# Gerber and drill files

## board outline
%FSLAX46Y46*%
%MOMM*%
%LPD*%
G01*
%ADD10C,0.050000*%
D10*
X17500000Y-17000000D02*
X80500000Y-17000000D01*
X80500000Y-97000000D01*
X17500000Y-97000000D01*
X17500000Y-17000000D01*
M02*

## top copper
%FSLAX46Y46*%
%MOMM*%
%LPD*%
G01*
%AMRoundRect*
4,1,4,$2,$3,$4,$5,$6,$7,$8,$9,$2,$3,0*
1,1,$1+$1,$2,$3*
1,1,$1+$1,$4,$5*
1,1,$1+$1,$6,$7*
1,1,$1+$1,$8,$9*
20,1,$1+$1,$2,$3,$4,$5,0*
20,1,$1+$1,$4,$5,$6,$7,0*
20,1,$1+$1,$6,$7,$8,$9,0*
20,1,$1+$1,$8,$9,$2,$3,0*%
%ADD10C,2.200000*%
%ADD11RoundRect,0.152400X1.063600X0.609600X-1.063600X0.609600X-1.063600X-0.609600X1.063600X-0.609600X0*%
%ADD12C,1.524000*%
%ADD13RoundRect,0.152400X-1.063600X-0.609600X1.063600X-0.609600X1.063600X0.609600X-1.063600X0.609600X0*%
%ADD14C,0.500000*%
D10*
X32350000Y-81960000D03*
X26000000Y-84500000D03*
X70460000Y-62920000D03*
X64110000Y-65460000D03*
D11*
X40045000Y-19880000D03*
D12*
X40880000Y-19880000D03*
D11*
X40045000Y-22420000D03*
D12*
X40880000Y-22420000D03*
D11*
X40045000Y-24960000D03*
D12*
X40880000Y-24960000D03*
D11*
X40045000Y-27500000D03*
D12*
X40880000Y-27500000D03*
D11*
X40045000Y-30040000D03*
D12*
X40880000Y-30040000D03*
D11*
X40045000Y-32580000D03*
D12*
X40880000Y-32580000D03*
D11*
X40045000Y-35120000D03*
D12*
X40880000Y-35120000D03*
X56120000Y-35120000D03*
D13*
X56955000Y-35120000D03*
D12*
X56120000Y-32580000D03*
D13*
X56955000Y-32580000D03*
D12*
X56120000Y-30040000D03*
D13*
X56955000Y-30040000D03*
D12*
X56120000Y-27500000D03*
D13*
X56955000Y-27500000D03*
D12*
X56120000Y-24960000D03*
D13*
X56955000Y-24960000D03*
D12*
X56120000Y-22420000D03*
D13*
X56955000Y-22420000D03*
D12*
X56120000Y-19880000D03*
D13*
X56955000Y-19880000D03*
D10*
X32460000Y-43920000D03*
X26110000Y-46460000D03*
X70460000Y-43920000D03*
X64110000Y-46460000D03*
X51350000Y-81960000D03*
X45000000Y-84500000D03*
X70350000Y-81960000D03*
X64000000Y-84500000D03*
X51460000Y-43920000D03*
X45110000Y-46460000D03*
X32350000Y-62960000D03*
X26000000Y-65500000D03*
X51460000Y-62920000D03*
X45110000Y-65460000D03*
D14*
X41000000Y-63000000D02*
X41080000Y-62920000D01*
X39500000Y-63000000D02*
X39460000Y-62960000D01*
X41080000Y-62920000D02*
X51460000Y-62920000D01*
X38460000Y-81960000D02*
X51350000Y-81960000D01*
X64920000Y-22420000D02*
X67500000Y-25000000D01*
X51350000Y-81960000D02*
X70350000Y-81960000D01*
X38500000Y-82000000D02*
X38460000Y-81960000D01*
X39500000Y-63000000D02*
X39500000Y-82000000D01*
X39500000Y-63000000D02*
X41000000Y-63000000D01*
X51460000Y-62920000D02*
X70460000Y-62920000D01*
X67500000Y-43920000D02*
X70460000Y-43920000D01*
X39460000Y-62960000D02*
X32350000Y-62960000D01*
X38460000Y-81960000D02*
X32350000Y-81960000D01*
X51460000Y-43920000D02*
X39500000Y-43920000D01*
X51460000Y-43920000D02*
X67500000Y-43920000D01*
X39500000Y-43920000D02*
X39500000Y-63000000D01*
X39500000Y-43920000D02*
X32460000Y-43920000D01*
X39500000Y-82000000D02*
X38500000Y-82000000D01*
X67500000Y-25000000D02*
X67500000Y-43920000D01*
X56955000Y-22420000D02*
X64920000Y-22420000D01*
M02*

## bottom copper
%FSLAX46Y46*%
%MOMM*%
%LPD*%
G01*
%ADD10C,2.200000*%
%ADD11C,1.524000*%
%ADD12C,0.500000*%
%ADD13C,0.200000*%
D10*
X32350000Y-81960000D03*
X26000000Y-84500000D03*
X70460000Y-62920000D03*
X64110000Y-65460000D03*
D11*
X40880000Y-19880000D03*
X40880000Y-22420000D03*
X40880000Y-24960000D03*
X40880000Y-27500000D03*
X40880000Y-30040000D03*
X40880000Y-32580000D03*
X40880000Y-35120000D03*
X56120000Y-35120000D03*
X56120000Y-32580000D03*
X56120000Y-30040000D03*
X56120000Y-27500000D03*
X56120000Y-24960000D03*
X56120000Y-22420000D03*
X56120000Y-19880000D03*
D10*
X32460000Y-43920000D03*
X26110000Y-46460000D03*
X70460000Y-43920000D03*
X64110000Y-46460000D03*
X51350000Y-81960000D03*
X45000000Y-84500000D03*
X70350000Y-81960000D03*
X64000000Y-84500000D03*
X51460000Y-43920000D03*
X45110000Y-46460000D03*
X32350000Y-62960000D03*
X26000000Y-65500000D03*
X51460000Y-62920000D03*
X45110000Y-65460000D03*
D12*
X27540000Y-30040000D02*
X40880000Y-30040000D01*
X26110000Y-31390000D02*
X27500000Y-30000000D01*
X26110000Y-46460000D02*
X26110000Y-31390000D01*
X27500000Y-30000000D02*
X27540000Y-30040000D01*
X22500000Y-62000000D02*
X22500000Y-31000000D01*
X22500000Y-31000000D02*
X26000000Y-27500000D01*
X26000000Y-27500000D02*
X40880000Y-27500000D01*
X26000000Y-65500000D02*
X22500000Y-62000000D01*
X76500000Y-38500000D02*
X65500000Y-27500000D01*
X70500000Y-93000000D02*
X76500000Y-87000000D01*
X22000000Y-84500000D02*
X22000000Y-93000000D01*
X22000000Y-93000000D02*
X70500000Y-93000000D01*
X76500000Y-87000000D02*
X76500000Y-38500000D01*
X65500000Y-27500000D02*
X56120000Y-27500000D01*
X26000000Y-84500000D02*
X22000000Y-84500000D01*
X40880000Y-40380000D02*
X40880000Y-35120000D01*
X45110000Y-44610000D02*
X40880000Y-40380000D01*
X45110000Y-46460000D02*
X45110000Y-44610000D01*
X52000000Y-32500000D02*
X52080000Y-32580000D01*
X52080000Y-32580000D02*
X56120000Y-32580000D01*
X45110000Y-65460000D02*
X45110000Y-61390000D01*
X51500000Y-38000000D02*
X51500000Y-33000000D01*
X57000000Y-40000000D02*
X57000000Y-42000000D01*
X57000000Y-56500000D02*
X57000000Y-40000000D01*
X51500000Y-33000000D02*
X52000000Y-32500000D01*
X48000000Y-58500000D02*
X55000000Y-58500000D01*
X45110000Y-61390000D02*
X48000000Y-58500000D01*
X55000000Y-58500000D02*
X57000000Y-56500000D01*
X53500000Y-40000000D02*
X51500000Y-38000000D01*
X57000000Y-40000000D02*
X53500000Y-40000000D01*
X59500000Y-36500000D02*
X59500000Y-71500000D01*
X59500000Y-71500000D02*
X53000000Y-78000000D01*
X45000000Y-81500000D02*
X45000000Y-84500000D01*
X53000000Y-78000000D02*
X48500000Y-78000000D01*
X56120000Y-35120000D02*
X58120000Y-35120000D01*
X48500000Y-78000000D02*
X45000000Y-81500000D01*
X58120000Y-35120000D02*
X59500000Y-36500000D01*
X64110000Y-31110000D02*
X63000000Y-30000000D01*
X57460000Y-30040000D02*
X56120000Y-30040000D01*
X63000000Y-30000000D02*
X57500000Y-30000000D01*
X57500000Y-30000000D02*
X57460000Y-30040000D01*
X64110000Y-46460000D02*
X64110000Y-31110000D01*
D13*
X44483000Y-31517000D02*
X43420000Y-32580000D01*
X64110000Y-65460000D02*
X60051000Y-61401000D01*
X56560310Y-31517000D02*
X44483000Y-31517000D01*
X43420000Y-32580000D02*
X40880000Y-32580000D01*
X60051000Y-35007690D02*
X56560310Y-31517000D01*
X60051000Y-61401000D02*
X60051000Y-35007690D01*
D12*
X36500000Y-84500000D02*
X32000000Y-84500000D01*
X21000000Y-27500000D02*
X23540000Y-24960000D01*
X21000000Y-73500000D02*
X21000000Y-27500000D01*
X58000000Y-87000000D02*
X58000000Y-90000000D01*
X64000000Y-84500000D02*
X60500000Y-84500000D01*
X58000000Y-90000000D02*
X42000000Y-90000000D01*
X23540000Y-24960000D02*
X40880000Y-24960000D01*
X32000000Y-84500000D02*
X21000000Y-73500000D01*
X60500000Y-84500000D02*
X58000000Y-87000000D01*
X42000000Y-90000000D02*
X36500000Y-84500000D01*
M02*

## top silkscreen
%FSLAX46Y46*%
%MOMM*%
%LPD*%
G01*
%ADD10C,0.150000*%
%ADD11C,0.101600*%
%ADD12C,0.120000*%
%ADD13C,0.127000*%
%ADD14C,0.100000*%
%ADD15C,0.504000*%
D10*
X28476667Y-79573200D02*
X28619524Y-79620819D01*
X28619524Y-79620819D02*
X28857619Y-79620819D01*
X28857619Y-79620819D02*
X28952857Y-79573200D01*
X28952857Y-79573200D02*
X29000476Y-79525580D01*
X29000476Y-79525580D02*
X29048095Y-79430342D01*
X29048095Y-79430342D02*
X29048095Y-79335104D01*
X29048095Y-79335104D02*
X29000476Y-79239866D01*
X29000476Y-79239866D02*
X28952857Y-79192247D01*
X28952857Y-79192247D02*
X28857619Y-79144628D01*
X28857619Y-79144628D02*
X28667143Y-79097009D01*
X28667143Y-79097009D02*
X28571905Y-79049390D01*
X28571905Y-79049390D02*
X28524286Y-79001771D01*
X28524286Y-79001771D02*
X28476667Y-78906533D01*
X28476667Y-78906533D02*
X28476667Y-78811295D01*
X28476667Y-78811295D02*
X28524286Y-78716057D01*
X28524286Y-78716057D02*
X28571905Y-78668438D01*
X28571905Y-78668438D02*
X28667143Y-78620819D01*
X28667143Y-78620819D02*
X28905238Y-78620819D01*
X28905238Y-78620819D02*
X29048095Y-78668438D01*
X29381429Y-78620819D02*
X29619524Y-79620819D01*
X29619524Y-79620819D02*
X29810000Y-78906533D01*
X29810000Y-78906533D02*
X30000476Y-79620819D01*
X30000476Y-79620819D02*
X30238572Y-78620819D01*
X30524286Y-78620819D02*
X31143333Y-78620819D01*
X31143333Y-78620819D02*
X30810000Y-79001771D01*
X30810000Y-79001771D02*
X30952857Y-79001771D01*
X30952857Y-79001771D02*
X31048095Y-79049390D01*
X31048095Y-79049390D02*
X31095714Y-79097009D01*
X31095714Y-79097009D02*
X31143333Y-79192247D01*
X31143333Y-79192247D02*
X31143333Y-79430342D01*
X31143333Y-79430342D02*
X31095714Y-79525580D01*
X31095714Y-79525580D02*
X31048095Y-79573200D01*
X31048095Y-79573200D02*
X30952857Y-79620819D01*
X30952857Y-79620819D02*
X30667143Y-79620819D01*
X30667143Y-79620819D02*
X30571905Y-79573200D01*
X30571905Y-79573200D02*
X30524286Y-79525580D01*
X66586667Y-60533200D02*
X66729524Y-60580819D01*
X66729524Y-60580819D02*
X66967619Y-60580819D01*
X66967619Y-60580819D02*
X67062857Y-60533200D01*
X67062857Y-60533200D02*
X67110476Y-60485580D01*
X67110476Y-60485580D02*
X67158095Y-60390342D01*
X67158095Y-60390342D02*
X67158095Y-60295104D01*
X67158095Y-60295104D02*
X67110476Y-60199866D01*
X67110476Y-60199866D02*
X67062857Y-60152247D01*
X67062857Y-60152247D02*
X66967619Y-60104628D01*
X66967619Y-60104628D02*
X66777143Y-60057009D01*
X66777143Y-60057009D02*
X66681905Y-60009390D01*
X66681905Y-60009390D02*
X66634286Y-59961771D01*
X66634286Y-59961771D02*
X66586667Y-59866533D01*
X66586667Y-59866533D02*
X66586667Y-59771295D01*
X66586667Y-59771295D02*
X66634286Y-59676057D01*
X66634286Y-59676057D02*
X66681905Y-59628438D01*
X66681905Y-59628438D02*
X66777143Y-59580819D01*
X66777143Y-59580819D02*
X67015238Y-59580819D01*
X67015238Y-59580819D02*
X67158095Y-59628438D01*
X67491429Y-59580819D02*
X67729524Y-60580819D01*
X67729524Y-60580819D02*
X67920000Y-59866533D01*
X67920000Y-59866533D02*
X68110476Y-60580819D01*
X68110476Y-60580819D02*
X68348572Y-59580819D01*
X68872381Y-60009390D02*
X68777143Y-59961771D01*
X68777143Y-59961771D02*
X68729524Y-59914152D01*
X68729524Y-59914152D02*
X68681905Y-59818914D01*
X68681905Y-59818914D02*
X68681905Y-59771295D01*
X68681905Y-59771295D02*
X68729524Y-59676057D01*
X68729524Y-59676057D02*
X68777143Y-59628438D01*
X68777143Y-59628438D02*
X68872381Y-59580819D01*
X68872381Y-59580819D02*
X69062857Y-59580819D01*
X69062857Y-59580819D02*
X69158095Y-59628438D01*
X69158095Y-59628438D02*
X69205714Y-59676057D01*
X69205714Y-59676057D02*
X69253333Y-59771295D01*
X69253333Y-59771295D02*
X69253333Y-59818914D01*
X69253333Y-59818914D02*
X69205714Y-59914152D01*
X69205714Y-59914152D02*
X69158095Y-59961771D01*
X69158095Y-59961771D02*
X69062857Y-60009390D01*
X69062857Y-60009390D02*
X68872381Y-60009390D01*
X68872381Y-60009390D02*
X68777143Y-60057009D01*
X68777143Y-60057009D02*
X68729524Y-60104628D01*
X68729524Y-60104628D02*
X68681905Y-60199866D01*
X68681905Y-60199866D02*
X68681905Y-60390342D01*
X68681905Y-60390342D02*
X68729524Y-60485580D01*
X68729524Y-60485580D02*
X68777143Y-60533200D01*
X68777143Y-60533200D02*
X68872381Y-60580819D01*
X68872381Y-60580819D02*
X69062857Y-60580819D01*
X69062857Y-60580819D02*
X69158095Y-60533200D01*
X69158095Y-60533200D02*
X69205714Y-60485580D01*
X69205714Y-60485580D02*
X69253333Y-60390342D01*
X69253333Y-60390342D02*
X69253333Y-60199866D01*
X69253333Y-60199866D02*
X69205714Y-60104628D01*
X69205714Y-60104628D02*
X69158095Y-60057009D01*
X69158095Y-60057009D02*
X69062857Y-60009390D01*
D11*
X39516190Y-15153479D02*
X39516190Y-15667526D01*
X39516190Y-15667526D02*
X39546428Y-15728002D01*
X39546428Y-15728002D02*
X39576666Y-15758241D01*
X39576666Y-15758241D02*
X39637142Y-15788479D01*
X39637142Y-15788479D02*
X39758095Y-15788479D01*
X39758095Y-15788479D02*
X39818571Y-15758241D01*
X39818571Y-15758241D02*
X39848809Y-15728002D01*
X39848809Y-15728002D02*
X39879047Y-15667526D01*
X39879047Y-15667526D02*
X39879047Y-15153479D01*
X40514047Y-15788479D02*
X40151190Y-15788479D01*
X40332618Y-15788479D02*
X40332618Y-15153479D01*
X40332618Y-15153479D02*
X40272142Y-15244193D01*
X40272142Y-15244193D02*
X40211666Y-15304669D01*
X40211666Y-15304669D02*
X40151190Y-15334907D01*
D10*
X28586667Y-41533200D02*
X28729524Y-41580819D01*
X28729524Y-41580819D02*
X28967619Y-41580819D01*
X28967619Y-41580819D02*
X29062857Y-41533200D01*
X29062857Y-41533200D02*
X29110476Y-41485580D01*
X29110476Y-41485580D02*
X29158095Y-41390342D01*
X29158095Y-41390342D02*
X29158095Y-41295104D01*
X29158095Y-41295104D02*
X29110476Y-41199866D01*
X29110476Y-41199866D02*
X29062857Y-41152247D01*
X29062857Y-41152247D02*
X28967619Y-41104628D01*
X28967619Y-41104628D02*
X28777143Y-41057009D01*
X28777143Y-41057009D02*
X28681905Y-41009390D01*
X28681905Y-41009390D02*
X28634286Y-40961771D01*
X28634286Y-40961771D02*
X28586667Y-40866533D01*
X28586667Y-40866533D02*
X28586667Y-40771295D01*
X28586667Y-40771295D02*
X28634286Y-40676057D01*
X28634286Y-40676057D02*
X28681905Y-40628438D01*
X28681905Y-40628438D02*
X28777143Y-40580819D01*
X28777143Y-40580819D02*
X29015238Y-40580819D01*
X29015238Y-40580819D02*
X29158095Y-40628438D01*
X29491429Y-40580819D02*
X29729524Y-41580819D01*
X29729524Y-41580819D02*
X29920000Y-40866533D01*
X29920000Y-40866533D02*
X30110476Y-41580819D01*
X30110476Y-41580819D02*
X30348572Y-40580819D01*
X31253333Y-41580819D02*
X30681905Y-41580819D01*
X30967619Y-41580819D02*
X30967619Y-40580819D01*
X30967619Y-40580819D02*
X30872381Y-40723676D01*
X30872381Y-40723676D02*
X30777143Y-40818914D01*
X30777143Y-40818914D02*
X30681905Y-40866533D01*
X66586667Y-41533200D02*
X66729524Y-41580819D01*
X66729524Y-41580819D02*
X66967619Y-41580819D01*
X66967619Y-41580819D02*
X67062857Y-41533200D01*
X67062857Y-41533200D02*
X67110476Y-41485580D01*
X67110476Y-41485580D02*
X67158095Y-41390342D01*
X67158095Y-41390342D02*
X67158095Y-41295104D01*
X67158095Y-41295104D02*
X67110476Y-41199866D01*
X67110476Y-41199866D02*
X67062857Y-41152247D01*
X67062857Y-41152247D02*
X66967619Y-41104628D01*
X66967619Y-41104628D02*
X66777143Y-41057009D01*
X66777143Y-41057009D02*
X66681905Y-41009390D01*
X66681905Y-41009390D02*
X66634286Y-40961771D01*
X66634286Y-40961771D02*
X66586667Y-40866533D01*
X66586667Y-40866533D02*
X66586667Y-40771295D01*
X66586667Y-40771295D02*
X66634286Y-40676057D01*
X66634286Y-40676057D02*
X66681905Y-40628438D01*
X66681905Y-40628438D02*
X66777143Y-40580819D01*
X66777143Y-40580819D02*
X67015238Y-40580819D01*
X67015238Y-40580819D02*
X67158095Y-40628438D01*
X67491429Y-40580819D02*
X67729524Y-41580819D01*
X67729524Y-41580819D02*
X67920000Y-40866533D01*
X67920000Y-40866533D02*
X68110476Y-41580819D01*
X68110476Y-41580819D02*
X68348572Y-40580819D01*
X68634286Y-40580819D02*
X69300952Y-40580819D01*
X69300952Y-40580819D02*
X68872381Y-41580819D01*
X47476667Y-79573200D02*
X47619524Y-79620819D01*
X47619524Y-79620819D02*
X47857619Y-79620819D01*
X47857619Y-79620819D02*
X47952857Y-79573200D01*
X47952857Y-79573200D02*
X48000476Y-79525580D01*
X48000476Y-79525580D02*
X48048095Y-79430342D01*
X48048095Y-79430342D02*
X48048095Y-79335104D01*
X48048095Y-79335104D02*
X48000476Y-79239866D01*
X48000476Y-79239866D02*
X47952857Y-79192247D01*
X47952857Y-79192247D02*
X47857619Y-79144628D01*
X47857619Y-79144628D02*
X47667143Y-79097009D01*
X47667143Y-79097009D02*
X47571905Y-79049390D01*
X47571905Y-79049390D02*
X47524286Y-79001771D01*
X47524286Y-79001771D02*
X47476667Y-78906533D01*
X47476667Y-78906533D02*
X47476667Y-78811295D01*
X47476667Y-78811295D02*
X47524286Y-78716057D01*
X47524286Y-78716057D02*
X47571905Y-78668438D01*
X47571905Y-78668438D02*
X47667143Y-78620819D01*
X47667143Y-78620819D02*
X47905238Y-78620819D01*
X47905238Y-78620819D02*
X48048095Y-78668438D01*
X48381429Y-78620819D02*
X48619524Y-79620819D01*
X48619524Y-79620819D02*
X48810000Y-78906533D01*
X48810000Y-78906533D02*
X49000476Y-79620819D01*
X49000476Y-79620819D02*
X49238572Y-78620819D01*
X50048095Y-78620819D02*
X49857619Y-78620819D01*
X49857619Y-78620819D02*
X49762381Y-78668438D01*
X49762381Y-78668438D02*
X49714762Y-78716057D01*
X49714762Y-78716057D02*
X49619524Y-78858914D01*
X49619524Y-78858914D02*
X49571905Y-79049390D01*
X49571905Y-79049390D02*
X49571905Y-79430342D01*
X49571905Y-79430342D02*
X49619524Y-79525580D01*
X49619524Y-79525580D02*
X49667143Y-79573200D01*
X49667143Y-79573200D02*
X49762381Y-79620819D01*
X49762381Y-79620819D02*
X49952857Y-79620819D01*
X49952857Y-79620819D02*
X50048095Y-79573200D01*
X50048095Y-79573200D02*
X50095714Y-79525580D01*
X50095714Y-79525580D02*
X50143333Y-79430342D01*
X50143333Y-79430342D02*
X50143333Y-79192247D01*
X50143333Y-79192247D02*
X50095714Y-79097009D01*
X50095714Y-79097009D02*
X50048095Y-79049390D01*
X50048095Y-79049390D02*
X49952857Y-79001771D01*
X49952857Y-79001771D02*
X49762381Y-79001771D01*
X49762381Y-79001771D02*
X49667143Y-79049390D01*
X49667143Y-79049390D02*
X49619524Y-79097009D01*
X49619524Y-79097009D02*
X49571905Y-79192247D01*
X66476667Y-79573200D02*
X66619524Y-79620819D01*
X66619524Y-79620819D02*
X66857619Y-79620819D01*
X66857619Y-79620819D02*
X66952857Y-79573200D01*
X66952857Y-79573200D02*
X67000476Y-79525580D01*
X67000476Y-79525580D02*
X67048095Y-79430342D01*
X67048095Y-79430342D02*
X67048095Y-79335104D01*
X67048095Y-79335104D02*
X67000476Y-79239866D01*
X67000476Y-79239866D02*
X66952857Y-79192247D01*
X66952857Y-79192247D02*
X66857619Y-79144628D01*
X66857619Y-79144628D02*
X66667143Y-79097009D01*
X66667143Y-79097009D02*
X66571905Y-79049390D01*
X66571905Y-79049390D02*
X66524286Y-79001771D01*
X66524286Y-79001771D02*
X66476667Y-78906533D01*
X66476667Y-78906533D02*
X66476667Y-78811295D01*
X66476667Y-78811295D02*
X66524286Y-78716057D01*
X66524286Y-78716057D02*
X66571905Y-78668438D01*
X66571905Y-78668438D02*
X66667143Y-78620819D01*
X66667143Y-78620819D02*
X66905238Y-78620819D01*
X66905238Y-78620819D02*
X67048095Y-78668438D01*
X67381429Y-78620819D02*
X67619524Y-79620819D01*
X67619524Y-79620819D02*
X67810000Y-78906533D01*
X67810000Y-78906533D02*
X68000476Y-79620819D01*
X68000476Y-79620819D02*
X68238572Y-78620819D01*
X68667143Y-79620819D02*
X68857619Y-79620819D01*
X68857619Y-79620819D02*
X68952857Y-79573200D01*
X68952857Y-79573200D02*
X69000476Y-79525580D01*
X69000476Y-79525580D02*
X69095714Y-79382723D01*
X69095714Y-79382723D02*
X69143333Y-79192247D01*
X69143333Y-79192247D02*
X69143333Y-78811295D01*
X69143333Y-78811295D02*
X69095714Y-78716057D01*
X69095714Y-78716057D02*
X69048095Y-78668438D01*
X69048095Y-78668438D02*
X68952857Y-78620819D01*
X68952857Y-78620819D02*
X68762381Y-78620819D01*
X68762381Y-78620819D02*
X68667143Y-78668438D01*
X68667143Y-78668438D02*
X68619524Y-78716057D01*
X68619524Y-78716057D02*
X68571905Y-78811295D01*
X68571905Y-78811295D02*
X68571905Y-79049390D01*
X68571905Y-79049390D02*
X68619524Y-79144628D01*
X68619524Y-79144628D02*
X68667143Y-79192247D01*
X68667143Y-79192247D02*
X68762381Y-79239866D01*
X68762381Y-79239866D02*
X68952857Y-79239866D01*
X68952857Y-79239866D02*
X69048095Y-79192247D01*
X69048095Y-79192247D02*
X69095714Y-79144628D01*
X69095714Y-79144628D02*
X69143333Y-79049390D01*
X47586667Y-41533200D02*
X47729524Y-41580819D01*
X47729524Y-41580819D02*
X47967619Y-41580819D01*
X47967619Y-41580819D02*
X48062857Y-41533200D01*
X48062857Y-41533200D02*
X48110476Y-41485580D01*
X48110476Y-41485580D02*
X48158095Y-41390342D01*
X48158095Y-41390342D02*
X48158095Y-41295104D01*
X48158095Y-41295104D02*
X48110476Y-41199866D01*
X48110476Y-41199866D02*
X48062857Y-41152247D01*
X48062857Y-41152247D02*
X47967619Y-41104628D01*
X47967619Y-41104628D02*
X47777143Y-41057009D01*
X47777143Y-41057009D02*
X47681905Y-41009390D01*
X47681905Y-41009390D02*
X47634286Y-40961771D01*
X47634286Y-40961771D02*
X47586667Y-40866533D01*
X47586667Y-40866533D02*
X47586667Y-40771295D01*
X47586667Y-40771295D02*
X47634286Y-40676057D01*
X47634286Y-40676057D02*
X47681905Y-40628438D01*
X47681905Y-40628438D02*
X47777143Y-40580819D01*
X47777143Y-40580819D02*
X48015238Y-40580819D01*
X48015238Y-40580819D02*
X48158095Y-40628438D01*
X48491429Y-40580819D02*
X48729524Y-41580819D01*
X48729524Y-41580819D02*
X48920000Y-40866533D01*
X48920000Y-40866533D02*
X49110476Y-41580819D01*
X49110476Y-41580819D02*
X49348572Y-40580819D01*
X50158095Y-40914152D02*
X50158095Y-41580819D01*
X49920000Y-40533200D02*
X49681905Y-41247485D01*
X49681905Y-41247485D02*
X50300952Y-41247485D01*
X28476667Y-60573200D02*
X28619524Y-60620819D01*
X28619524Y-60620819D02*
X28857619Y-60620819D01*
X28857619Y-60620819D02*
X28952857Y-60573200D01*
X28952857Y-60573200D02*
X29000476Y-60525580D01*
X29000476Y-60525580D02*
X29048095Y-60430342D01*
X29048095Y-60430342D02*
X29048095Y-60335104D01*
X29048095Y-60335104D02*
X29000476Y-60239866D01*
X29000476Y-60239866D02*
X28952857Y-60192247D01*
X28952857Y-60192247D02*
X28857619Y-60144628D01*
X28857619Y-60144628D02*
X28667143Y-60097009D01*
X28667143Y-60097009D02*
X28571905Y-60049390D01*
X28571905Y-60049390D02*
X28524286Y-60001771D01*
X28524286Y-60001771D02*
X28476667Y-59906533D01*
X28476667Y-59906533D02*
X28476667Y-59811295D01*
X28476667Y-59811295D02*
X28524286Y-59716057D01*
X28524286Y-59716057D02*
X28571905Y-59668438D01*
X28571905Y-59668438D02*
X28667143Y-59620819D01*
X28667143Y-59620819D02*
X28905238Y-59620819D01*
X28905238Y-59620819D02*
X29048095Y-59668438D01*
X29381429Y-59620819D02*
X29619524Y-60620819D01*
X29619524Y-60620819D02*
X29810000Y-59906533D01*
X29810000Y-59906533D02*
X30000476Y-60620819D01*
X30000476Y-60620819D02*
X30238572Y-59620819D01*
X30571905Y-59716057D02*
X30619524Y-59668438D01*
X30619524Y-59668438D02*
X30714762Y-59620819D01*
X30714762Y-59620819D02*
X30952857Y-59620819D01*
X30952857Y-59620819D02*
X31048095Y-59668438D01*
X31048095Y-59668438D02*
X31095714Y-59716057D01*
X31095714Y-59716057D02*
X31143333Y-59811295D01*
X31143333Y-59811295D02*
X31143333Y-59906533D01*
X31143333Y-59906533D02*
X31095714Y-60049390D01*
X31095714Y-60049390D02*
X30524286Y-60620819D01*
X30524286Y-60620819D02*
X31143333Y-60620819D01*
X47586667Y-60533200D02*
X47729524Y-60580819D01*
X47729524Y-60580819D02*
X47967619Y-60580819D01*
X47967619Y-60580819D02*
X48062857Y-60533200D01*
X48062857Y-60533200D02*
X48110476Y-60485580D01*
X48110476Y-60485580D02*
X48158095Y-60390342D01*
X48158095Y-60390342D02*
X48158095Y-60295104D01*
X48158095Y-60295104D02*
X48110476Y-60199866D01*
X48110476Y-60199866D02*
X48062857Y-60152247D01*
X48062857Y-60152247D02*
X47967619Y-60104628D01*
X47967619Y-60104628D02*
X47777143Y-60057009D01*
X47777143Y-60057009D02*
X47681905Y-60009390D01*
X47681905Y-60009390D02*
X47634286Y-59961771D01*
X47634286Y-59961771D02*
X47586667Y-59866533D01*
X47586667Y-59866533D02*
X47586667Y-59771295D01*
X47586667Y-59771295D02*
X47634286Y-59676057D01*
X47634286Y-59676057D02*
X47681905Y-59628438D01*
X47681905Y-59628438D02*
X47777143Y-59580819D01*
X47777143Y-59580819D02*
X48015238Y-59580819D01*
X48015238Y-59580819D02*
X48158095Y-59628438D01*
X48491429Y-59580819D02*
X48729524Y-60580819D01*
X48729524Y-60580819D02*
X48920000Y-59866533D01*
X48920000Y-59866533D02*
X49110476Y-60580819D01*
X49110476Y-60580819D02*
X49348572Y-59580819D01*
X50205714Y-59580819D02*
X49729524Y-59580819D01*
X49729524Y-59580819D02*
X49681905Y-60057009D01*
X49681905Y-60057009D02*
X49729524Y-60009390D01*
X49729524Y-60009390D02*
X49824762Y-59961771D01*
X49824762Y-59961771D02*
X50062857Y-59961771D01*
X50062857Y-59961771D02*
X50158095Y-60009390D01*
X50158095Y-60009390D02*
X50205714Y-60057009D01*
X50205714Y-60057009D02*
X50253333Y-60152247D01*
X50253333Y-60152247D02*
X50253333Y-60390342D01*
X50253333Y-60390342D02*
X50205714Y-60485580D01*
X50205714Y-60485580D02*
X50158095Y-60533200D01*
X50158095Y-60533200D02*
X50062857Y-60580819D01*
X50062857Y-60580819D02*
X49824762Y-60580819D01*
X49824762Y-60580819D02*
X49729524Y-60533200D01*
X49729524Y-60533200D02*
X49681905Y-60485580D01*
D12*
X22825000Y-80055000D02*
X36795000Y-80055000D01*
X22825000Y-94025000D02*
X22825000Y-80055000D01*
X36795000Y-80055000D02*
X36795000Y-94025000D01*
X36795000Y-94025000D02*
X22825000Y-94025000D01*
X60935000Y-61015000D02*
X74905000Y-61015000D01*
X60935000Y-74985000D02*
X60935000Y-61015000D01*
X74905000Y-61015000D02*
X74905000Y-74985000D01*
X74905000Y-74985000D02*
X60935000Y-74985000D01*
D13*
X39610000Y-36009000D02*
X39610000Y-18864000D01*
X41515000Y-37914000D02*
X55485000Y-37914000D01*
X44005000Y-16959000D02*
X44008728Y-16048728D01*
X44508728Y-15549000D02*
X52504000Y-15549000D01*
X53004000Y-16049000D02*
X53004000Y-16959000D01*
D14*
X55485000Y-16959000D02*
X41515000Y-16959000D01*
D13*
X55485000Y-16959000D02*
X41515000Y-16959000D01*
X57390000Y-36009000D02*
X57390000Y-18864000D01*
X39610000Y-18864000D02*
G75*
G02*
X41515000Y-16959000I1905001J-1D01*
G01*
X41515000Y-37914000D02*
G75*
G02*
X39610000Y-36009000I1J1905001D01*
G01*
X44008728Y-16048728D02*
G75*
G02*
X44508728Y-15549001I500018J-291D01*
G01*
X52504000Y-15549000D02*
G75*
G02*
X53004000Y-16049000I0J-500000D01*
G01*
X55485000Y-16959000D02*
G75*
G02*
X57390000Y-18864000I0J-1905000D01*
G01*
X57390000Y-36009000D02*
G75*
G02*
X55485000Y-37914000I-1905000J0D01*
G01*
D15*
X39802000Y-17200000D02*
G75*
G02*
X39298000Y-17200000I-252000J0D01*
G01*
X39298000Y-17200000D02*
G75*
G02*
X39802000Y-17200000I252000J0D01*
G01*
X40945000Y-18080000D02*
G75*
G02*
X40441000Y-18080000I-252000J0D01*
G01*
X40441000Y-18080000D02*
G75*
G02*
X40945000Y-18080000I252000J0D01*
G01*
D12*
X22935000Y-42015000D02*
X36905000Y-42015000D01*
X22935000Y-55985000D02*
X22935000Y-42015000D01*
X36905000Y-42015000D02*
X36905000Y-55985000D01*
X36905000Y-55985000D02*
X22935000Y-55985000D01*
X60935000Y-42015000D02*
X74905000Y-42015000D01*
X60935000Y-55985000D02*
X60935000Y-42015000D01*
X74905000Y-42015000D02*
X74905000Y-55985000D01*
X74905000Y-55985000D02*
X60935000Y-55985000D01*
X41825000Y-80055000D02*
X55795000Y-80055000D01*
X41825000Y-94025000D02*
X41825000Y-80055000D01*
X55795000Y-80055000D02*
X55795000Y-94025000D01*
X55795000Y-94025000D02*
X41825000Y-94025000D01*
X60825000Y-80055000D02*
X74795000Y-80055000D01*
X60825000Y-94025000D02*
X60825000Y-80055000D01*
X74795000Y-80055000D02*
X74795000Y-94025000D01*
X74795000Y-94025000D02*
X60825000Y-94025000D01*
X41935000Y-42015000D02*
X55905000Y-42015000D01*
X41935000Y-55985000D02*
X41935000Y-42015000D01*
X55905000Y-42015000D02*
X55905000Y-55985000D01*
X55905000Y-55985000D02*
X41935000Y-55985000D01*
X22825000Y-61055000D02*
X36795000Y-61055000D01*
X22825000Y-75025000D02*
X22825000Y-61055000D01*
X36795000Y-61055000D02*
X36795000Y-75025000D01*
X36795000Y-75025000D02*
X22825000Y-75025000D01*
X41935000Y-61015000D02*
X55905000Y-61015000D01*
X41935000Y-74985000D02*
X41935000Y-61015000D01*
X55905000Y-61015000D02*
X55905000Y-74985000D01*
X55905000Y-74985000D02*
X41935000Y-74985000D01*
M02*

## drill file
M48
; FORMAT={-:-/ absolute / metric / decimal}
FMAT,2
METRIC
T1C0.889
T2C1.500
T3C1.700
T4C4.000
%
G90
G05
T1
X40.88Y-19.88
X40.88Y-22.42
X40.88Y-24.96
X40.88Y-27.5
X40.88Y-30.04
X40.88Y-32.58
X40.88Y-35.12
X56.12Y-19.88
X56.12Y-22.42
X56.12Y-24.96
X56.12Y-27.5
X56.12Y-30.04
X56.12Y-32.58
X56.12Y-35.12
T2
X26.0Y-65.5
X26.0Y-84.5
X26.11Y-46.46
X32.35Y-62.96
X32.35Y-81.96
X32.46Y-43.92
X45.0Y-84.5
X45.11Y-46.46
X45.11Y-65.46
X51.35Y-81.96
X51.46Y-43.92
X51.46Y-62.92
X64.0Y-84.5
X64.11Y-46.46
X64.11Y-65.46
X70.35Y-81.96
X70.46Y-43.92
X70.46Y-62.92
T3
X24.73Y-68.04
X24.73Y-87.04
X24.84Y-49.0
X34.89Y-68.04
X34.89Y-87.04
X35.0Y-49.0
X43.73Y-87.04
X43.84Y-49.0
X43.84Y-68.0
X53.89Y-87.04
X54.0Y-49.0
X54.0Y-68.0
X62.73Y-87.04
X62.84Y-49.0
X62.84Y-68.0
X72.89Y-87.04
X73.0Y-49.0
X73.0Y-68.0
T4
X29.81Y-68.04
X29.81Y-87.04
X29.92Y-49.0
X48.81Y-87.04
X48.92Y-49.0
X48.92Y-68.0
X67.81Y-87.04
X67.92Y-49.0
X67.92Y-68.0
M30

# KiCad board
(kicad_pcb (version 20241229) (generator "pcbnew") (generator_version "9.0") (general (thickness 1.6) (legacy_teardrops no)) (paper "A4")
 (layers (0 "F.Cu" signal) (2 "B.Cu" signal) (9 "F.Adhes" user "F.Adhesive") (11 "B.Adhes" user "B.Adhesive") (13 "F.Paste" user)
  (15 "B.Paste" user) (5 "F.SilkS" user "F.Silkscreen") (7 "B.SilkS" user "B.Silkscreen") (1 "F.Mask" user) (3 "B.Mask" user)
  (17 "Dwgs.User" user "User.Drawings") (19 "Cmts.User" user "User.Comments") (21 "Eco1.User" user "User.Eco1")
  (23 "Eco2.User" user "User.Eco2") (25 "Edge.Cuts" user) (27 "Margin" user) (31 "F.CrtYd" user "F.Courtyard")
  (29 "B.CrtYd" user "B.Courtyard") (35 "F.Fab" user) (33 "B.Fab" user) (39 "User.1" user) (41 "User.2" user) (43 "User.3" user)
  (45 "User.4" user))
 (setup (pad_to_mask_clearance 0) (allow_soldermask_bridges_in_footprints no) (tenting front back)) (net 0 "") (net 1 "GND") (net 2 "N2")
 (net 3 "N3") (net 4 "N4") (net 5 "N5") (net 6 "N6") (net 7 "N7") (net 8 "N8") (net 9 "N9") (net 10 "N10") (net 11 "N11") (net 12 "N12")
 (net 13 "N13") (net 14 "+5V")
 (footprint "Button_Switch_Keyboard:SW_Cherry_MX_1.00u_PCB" (layer "F.Cu") (at 32.35 81.96)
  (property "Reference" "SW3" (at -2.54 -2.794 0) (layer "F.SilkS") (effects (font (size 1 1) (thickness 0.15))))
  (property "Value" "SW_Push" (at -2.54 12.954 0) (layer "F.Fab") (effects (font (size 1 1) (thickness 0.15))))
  (fp_line (start -9.525 -1.905) (end 4.445 -1.905) (stroke (width 0.12) (type solid)) (layer "F.SilkS"))
  (fp_line (start -9.525 12.065) (end -9.525 -1.905) (stroke (width 0.12) (type solid)) (layer "F.SilkS"))
  (fp_line (start 4.445 -1.905) (end 4.445 12.065) (stroke (width 0.12) (type solid)) (layer "F.SilkS"))
  (fp_line (start 4.445 12.065) (end -9.525 12.065) (stroke (width 0.12) (type solid)) (layer "F.SilkS"))
  (pad "" np_thru_hole circle (at -7.62 5.08) (size 1.7 1.7) (drill 1.7) (layers "*.Cu" "*.Mask"))
  (pad "" np_thru_hole circle (at -2.54 5.08) (size 4 4) (drill 4) (layers "*.Cu" "*.Mask"))
  (pad "" np_thru_hole circle (at 2.54 5.08) (size 1.7 1.7) (drill 1.7) (layers "*.Cu" "*.Mask"))
  (pad "1" thru_hole circle (at 0 0) (size 2.2 2.2) (drill 1.5) (layers "*.Cu" "*.Mask") (remove_unused_layers no) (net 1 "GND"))
  (pad "2" thru_hole circle (at -6.35 2.54) (size 2.2 2.2) (drill 1.5) (layers "*.Cu" "*.Mask") (remove_unused_layers no) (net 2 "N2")))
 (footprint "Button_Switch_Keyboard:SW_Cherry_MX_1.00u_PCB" (layer "F.Cu") (at 70.46 62.92)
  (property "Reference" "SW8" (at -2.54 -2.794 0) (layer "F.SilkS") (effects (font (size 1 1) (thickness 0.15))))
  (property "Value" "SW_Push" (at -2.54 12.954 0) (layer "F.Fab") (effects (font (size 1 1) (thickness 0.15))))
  (fp_line (start -9.525 -1.905) (end 4.445 -1.905) (stroke (width 0.12) (type solid)) (layer "F.SilkS"))
  (fp_line (start -9.525 12.065) (end -9.525 -1.905) (stroke (width 0.12) (type solid)) (layer "F.SilkS"))
  (fp_line (start 4.445 -1.905) (end 4.445 12.065) (stroke (width 0.12) (type solid)) (layer "F.SilkS"))
  (fp_line (start 4.445 12.065) (end -9.525 12.065) (stroke (width 0.12) (type solid)) (layer "F.SilkS"))
  (pad "" np_thru_hole circle (at -7.62 5.08) (size 1.7 1.7) (drill 1.7) (layers "*.Cu" "*.Mask"))
  (pad "" np_thru_hole circle (at -2.54 5.08) (size 4 4) (drill 4) (layers "*.Cu" "*.Mask"))
  (pad "" np_thru_hole circle (at 2.54 5.08) (size 1.7 1.7) (drill 1.7) (layers "*.Cu" "*.Mask"))
  (pad "1" thru_hole circle (at 0 0) (size 2.2 2.2) (drill 1.5) (layers "*.Cu" "*.Mask") (remove_unused_layers no) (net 1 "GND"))
  (pad "2" thru_hole circle (at -6.35 2.54) (size 2.2 2.2) (drill 1.5) (layers "*.Cu" "*.Mask") (remove_unused_layers no) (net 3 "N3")))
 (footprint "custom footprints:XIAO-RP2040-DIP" (layer "F.Cu") (at 48.5 27.5)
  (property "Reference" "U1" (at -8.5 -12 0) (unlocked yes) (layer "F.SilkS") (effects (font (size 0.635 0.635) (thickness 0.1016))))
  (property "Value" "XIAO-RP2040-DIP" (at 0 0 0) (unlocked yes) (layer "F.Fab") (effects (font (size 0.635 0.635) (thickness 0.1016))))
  (fp_line (start -8.89 8.509) (end -8.89 -8.636) (stroke (width 0.127) (type solid)) (layer "F.SilkS"))
  (fp_line (start -6.985 10.414) (end 6.985 10.414) (stroke (width 0.127) (type solid)) (layer "F.SilkS"))
  (fp_line (start -4.495 -10.541) (end -4.491272 -11.451272) (stroke (width 0.127) (type solid)) (layer "F.SilkS"))
  (fp_line (start -3.991272 -11.951) (end 4.004 -11.951) (stroke (width 0.127) (type solid)) (layer "F.SilkS"))
  (fp_line (start 4.504 -11.451) (end 4.504 -10.541) (stroke (width 0.127) (type solid)) (layer "F.SilkS"))
  (fp_line (start 6.985 -10.541) (end -6.985 -10.541) (stroke (width 0.1) (type solid)) (layer "F.SilkS"))
  (fp_line (start 6.985 -10.541) (end -6.985 -10.541) (stroke (width 0.127) (type solid)) (layer "F.SilkS"))
  (fp_line (start 8.89 8.509) (end 8.89 -8.636) (stroke (width 0.127) (type solid)) (layer "F.SilkS"))
  (fp_arc (start -8.89 -8.636) (mid -8.332038 -9.983038) (end -6.985 -10.541) (stroke (width 0.127) (type solid)) (layer "F.SilkS"))
  (fp_arc (start -6.985 10.414) (mid -8.332038 9.856038) (end -8.89 8.509) (stroke (width 0.127) (type solid)) (layer "F.SilkS"))
  (fp_arc (start -4.491272 -11.451272) (mid -4.344728 -11.80464) (end -3.991272 -11.951) (stroke (width 0.127) (type default))
   (layer "F.SilkS"))
  (fp_arc (start 4.004 -11.951) (mid 4.357553 -11.804553) (end 4.504 -11.451) (stroke (width 0.127) (type default)) (layer "F.SilkS"))
  (fp_arc (start 6.985 -10.541) (mid 8.332038 -9.983038) (end 8.89 -8.636) (stroke (width 0.127) (type solid)) (layer "F.SilkS"))
  (fp_arc (start 8.89 8.509) (mid 8.332038 9.856038) (end 6.985 10.414) (stroke (width 0.127) (type solid)) (layer "F.SilkS"))
  (fp_circle (center -8.95 -10.3) (end -8.95 -10.554) (stroke (width 0.5) (type solid)) (fill yes) (layer "F.SilkS"))
  (fp_circle (center -7.807 -9.42) (end -7.807 -9.674) (stroke (width 0.5) (type solid)) (fill yes) (layer "F.SilkS"))
  (pad "1" smd roundrect (at -8.455 -7.62 180) (size 2.432 1.524) (layers "F.Cu" "F.Mask") (roundrect_rratio 0.1) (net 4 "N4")
   (thermal_bridge_angle 45))
  (pad "1" thru_hole circle (at -7.62 -7.62 180) (size 1.524 1.524) (drill 0.889) (layers "*.Cu" "*.Mask") (remove_unused_layers no)
   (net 4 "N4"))
  (pad "2" smd roundrect (at -8.455 -5.08 180) (size 2.432 1.524) (layers "F.Cu" "F.Mask") (roundrect_rratio 0.1) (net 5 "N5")
   (thermal_bridge_angle 45))
  (pad "2" thru_hole circle (at -7.62 -5.08 180) (size 1.524 1.524) (drill 0.889) (layers "*.Cu" "*.Mask") (remove_unused_layers no)
   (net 5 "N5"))
  (pad "3" smd roundrect (at -8.455 -2.54 180) (size 2.432 1.524) (layers "F.Cu" "F.Mask") (roundrect_rratio 0.1) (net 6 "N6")
   (thermal_bridge_angle 45))
  (pad "3" thru_hole circle (at -7.62 -2.54 180) (size 1.524 1.524) (drill 0.889) (layers "*.Cu" "*.Mask") (remove_unused_layers no)
   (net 6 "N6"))
  (pad "4" smd roundrect (at -8.455 0 180) (size 2.432 1.524) (layers "F.Cu" "F.Mask") (roundrect_rratio 0.1) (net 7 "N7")
   (thermal_bridge_angle 45))
  (pad "4" thru_hole circle (at -7.62 0 180) (size 1.524 1.524) (drill 0.889) (layers "*.Cu" "*.Mask") (remove_unused_layers no)
   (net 7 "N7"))
  (pad "5" smd roundrect (at -8.455 2.54 180) (size 2.432 1.524) (layers "F.Cu" "F.Mask") (roundrect_rratio 0.1) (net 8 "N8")
   (thermal_bridge_angle 45))
  (pad "5" thru_hole circle (at -7.62 2.54 180) (size 1.524 1.524) (drill 0.889) (layers "*.Cu" "*.Mask") (remove_unused_layers no)
   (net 8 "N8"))
  (pad "6" smd roundrect (at -8.455 5.08 180) (size 2.432 1.524) (layers "F.Cu" "F.Mask") (roundrect_rratio 0.1) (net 3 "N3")
   (thermal_bridge_angle 45))
  (pad "6" thru_hole circle (at -7.62 5.08 180) (size 1.524 1.524) (drill 0.889) (layers "*.Cu" "*.Mask") (remove_unused_layers no)
   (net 3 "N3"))
  (pad "7" smd roundrect (at -8.455 7.62 180) (size 2.432 1.524) (layers "F.Cu" "F.Mask") (roundrect_rratio 0.1) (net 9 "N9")
   (thermal_bridge_angle 45))
  (pad "7" thru_hole circle (at -7.62 7.62 180) (size 1.524 1.524) (drill 0.889) (layers "*.Cu" "*.Mask") (remove_unused_layers no)
   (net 9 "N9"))
  (pad "8" thru_hole circle (at 7.62 7.62) (size 1.524 1.524) (drill 0.889) (layers "*.Cu" "*.Mask") (remove_unused_layers no)
   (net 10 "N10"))
  (pad "8" smd roundrect (at 8.455 7.62) (size 2.432 1.524) (layers "F.Cu" "F.Mask") (roundrect_rratio 0.1) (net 10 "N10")
   (thermal_bridge_angle 45))
  (pad "9" thru_hole circle (at 7.62 5.08) (size 1.524 1.524) (drill 0.889) (layers "*.Cu" "*.Mask") (remove_unused_layers no)
   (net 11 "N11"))
  (pad "9" smd roundrect (at 8.455 5.08) (size 2.432 1.524) (layers "F.Cu" "F.Mask") (roundrect_rratio 0.1) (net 11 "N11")
   (thermal_bridge_angle 45))
  (pad "10" thru_hole circle (at 7.62 2.54) (size 1.524 1.524) (drill 0.889) (layers "*.Cu" "*.Mask") (remove_unused_layers no)
   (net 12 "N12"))
  (pad "10" smd roundrect (at 8.455 2.54) (size 2.432 1.524) (layers "F.Cu" "F.Mask") (roundrect_rratio 0.1) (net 12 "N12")
   (thermal_bridge_angle 45))
  (pad "11" thru_hole circle (at 7.62 0) (size 1.524 1.524) (drill 0.889) (layers "*.Cu" "*.Mask") (remove_unused_layers no) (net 2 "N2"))
  (pad "11" smd roundrect (at 8.455 0) (size 2.432 1.524) (layers "F.Cu" "F.Mask") (roundrect_rratio 0.1) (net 2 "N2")
   (thermal_bridge_angle 45))
  (pad "12" thru_hole circle (at 7.62 -2.54) (size 1.524 1.524) (drill 0.889) (layers "*.Cu" "*.Mask") (remove_unused_layers no)
   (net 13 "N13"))
  (pad "12" smd roundrect (at 8.455 -2.54) (size 2.432 1.524) (layers "F.Cu" "F.Mask") (roundrect_rratio 0.1) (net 13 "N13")
   (thermal_bridge_angle 45))
  (pad "13" thru_hole circle (at 7.62 -5.08) (size 1.524 1.524) (drill 0.889) (layers "*.Cu" "*.Mask") (remove_unused_layers no)
   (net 1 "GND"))
  (pad "13" smd roundrect (at 8.455 -5.08) (size 2.432 1.524) (layers "F.Cu" "F.Mask") (roundrect_rratio 0.1) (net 1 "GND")
   (thermal_bridge_angle 45))
  (pad "14" thru_hole circle (at 7.62 -7.62) (size 1.524 1.524) (drill 0.889) (layers "*.Cu" "*.Mask") (remove_unused_layers no)
   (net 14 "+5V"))
  (pad "14" smd roundrect (at 8.455 -7.62) (size 2.432 1.524) (layers "F.Cu" "F.Mask") (roundrect_rratio 0.1) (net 14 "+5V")
   (thermal_bridge_angle 45)))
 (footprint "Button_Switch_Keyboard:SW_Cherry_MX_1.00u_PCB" (layer "F.Cu") (at 32.46 43.92)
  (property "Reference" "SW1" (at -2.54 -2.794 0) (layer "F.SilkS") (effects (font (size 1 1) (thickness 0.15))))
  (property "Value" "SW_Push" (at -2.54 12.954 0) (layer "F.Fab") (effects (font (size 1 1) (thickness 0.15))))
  (fp_line (start -9.525 -1.905) (end 4.445 -1.905) (stroke (width 0.12) (type solid)) (layer "F.SilkS"))
  (fp_line (start -9.525 12.065) (end -9.525 -1.905) (stroke (width 0.12) (type solid)) (layer "F.SilkS"))
  (fp_line (start 4.445 -1.905) (end 4.445 12.065) (stroke (width 0.12) (type solid)) (layer "F.SilkS"))
  (fp_line (start 4.445 12.065) (end -9.525 12.065) (stroke (width 0.12) (type solid)) (layer "F.SilkS"))
  (pad "" np_thru_hole circle (at -7.62 5.08) (size 1.7 1.7) (drill 1.7) (layers "*.Cu" "*.Mask"))
  (pad "" np_thru_hole circle (at -2.54 5.08) (size 4 4) (drill 4) (layers "*.Cu" "*.Mask"))
  (pad "" np_thru_hole circle (at 2.54 5.08) (size 1.7 1.7) (drill 1.7) (layers "*.Cu" "*.Mask"))
  (pad "1" thru_hole circle (at 0 0) (size 2.2 2.2) (drill 1.5) (layers "*.Cu" "*.Mask") (remove_unused_layers no) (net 1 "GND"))
  (pad "2" thru_hole circle (at -6.35 2.54) (size 2.2 2.2) (drill 1.5) (layers "*.Cu" "*.Mask") (remove_unused_layers no) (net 8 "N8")))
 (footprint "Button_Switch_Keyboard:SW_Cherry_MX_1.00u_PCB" (layer "F.Cu") (at 70.46 43.92)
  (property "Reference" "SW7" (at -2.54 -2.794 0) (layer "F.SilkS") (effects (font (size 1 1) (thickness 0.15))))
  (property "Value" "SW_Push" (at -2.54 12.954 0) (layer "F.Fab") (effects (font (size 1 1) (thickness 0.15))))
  (fp_line (start -9.525 -1.905) (end 4.445 -1.905) (stroke (width 0.12) (type solid)) (layer "F.SilkS"))
  (fp_line (start -9.525 12.065) (end -9.525 -1.905) (stroke (width 0.12) (type solid)) (layer "F.SilkS"))
  (fp_line (start 4.445 -1.905) (end 4.445 12.065) (stroke (width 0.12) (type solid)) (layer "F.SilkS"))
  (fp_line (start 4.445 12.065) (end -9.525 12.065) (stroke (width 0.12) (type solid)) (layer "F.SilkS"))
  (pad "" np_thru_hole circle (at -7.62 5.08) (size 1.7 1.7) (drill 1.7) (layers "*.Cu" "*.Mask"))
  (pad "" np_thru_hole circle (at -2.54 5.08) (size 4 4) (drill 4) (layers "*.Cu" "*.Mask"))
  (pad "" np_thru_hole circle (at 2.54 5.08) (size 1.7 1.7) (drill 1.7) (layers "*.Cu" "*.Mask"))
  (pad "1" thru_hole circle (at 0 0) (size 2.2 2.2) (drill 1.5) (layers "*.Cu" "*.Mask") (remove_unused_layers no) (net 1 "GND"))
  (pad "2" thru_hole circle (at -6.35 2.54) (size 2.2 2.2) (drill 1.5) (layers "*.Cu" "*.Mask") (remove_unused_layers no) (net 12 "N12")))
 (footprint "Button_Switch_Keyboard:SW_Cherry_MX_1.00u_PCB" (layer "F.Cu") (at 51.35 81.96)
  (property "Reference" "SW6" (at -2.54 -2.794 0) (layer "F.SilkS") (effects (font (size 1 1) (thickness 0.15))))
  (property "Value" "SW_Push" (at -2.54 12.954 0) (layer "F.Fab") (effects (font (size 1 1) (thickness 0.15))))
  (fp_line (start -9.525 -1.905) (end 4.445 -1.905) (stroke (width 0.12) (type solid)) (layer "F.SilkS"))
  (fp_line (start -9.525 12.065) (end -9.525 -1.905) (stroke (width 0.12) (type solid)) (layer "F.SilkS"))
  (fp_line (start 4.445 -1.905) (end 4.445 12.065) (stroke (width 0.12) (type solid)) (layer "F.SilkS"))
  (fp_line (start 4.445 12.065) (end -9.525 12.065) (stroke (width 0.12) (type solid)) (layer "F.SilkS"))
  (pad "" np_thru_hole circle (at -7.62 5.08) (size 1.7 1.7) (drill 1.7) (layers "*.Cu" "*.Mask"))
  (pad "" np_thru_hole circle (at -2.54 5.08) (size 4 4) (drill 4) (layers "*.Cu" "*.Mask"))
  (pad "" np_thru_hole circle (at 2.54 5.08) (size 1.7 1.7) (drill 1.7) (layers "*.Cu" "*.Mask"))
  (pad "1" thru_hole circle (at 0 0) (size 2.2 2.2) (drill 1.5) (layers "*.Cu" "*.Mask") (remove_unused_layers no) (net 1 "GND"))
  (pad "2" thru_hole circle (at -6.35 2.54) (size 2.2 2.2) (drill 1.5) (layers "*.Cu" "*.Mask") (remove_unused_layers no) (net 10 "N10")))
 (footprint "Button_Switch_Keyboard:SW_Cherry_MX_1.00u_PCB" (layer "F.Cu") (at 70.35 81.96)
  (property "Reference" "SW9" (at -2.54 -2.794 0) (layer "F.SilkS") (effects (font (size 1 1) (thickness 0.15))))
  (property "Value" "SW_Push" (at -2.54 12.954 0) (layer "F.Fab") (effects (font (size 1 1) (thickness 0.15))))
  (fp_line (start -9.525 -1.905) (end 4.445 -1.905) (stroke (width 0.12) (type solid)) (layer "F.SilkS"))
  (fp_line (start -9.525 12.065) (end -9.525 -1.905) (stroke (width 0.12) (type solid)) (layer "F.SilkS"))
  (fp_line (start 4.445 -1.905) (end 4.445 12.065) (stroke (width 0.12) (type solid)) (layer "F.SilkS"))
  (fp_line (start 4.445 12.065) (end -9.525 12.065) (stroke (width 0.12) (type solid)) (layer "F.SilkS"))
  (pad "" np_thru_hole circle (at -7.62 5.08) (size 1.7 1.7) (drill 1.7) (layers "*.Cu" "*.Mask"))
  (pad "" np_thru_hole circle (at -2.54 5.08) (size 4 4) (drill 4) (layers "*.Cu" "*.Mask"))
  (pad "" np_thru_hole circle (at 2.54 5.08) (size 1.7 1.7) (drill 1.7) (layers "*.Cu" "*.Mask"))
  (pad "1" thru_hole circle (at 0 0) (size 2.2 2.2) (drill 1.5) (layers "*.Cu" "*.Mask") (remove_unused_layers no) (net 1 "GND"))
  (pad "2" thru_hole circle (at -6.35 2.54) (size 2.2 2.2) (drill 1.5) (layers "*.Cu" "*.Mask") (remove_unused_layers no) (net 6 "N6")))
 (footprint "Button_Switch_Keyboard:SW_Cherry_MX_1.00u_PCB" (layer "F.Cu") (at 51.46 43.92)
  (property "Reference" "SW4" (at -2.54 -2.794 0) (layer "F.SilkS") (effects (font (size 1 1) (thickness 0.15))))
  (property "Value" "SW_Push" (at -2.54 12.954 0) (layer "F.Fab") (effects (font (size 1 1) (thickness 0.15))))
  (fp_line (start -9.525 -1.905) (end 4.445 -1.905) (stroke (width 0.12) (type solid)) (layer "F.SilkS"))
  (fp_line (start -9.525 12.065) (end -9.525 -1.905) (stroke (width 0.12) (type solid)) (layer "F.SilkS"))
  (fp_line (start 4.445 -1.905) (end 4.445 12.065) (stroke (width 0.12) (type solid)) (layer "F.SilkS"))
  (fp_line (start 4.445 12.065) (end -9.525 12.065) (stroke (width 0.12) (type solid)) (layer "F.SilkS"))
  (pad "" np_thru_hole circle (at -7.62 5.08) (size 1.7 1.7) (drill 1.7) (layers "*.Cu" "*.Mask"))
  (pad "" np_thru_hole circle (at -2.54 5.08) (size 4 4) (drill 4) (layers "*.Cu" "*.Mask"))
  (pad "" np_thru_hole circle (at 2.54 5.08) (size 1.7 1.7) (drill 1.7) (layers "*.Cu" "*.Mask"))
  (pad "1" thru_hole circle (at 0 0) (size 2.2 2.2) (drill 1.5) (layers "*.Cu" "*.Mask") (remove_unused_layers no) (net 1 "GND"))
  (pad "2" thru_hole circle (at -6.35 2.54) (size 2.2 2.2) (drill 1.5) (layers "*.Cu" "*.Mask") (remove_unused_layers no) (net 9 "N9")))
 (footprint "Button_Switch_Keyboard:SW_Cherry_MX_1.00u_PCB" (layer "F.Cu") (at 32.35 62.96)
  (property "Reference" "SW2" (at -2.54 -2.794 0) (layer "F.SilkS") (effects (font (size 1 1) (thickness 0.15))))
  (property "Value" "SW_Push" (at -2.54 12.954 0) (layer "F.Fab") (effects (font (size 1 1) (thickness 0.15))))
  (fp_line (start -9.525 -1.905) (end 4.445 -1.905) (stroke (width 0.12) (type solid)) (layer "F.SilkS"))
  (fp_line (start -9.525 12.065) (end -9.525 -1.905) (stroke (width 0.12) (type solid)) (layer "F.SilkS"))
  (fp_line (start 4.445 -1.905) (end 4.445 12.065) (stroke (width 0.12) (type solid)) (layer "F.SilkS"))
  (fp_line (start 4.445 12.065) (end -9.525 12.065) (stroke (width 0.12) (type solid)) (layer "F.SilkS"))
  (pad "" np_thru_hole circle (at -7.62 5.08) (size 1.7 1.7) (drill 1.7) (layers "*.Cu" "*.Mask"))
  (pad "" np_thru_hole circle (at -2.54 5.08) (size 4 4) (drill 4) (layers "*.Cu" "*.Mask"))
  (pad "" np_thru_hole circle (at 2.54 5.08) (size 1.7 1.7) (drill 1.7) (layers "*.Cu" "*.Mask"))
  (pad "1" thru_hole circle (at 0 0) (size 2.2 2.2) (drill 1.5) (layers "*.Cu" "*.Mask") (remove_unused_layers no) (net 1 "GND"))
  (pad "2" thru_hole circle (at -6.35 2.54) (size 2.2 2.2) (drill 1.5) (layers "*.Cu" "*.Mask") (remove_unused_layers no) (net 7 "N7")))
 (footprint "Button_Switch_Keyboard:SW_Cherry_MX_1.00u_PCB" (layer "F.Cu") (at 51.46 62.92)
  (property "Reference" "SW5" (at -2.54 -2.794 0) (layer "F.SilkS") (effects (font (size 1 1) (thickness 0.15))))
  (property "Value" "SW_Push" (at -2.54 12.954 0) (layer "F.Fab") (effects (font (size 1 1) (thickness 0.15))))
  (fp_line (start -9.525 -1.905) (end 4.445 -1.905) (stroke (width 0.12) (type solid)) (layer "F.SilkS"))
  (fp_line (start -9.525 12.065) (end -9.525 -1.905) (stroke (width 0.12) (type solid)) (layer "F.SilkS"))
  (fp_line (start 4.445 -1.905) (end 4.445 12.065) (stroke (width 0.12) (type solid)) (layer "F.SilkS"))
  (fp_line (start 4.445 12.065) (end -9.525 12.065) (stroke (width 0.12) (type solid)) (layer "F.SilkS"))
  (pad "" np_thru_hole circle (at -7.62 5.08) (size 1.7 1.7) (drill 1.7) (layers "*.Cu" "*.Mask"))
  (pad "" np_thru_hole circle (at -2.54 5.08) (size 4 4) (drill 4) (layers "*.Cu" "*.Mask"))
  (pad "" np_thru_hole circle (at 2.54 5.08) (size 1.7 1.7) (drill 1.7) (layers "*.Cu" "*.Mask"))
  (pad "1" thru_hole circle (at 0 0) (size 2.2 2.2) (drill 1.5) (layers "*.Cu" "*.Mask") (remove_unused_layers no) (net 1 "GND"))
  (pad "2" thru_hole circle (at -6.35 2.54) (size 2.2 2.2) (drill 1.5) (layers "*.Cu" "*.Mask") (remove_unused_layers no) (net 11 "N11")))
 (gr_rect (start 17.5 17) (end 80.5 97) (stroke (width 0.05) (type default)) (fill no) (layer "Edge.Cuts"))
 (segment (start 27.54 30.04) (end 40.88 30.04) (width 0.5) (layer "B.Cu") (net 8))
 (segment (start 26.11 31.39) (end 27.5 30) (width 0.5) (layer "B.Cu") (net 8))
 (segment (start 26.11 46.46) (end 26.11 31.39) (width 0.5) (layer "B.Cu") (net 8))
 (segment (start 27.5 30) (end 27.54 30.04) (width 0.5) (layer "B.Cu") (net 8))
 (segment (start 41 63) (end 41.08 62.92) (width 0.5) (layer "F.Cu") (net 1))
 (segment (start 39.5 63) (end 39.46 62.96) (width 0.5) (layer "F.Cu") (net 1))
 (segment (start 41.08 62.92) (end 51.46 62.92) (width 0.5) (layer "F.Cu") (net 1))
 (segment (start 38.46 81.96) (end 51.35 81.96) (width 0.5) (layer "F.Cu") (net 1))
 (segment (start 64.92 22.42) (end 67.5 25) (width 0.5) (layer "F.Cu") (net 1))
 (segment (start 51.35 81.96) (end 70.35 81.96) (width 0.5) (layer "F.Cu") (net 1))
 (segment (start 38.5 82) (end 38.46 81.96) (width 0.5) (layer "F.Cu") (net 1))
 (segment (start 39.5 63) (end 39.5 82) (width 0.5) (layer "F.Cu") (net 1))
 (segment (start 39.5 63) (end 41 63) (width 0.5) (layer "F.Cu") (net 1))
 (segment (start 51.46 62.92) (end 70.46 62.92) (width 0.5) (layer "F.Cu") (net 1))
 (segment (start 67.5 43.92) (end 70.46 43.92) (width 0.5) (layer "F.Cu") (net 1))
 (segment (start 39.46 62.96) (end 32.35 62.96) (width 0.5) (layer "F.Cu") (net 1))
 (segment (start 38.46 81.96) (end 32.35 81.96) (width 0.5) (layer "F.Cu") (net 1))
 (segment (start 51.46 43.92) (end 39.5 43.92) (width 0.5) (layer "F.Cu") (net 1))
 (segment (start 51.46 43.92) (end 67.5 43.92) (width 0.5) (layer "F.Cu") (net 1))
 (segment (start 39.5 43.92) (end 39.5 63) (width 0.5) (layer "F.Cu") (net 1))
 (segment (start 39.5 43.92) (end 32.46 43.92) (width 0.5) (layer "F.Cu") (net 1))
 (segment (start 39.5 82) (end 38.5 82) (width 0.5) (layer "F.Cu") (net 1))
 (segment (start 67.5 25) (end 67.5 43.92) (width 0.5) (layer "F.Cu") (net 1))
 (segment (start 56.955 22.42) (end 64.92 22.42) (width 0.5) (layer "F.Cu") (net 1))
 (segment (start 22.5 62) (end 22.5 31) (width 0.5) (layer "B.Cu") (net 7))
 (segment (start 22.5 31) (end 26 27.5) (width 0.5) (layer "B.Cu") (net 7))
 (segment (start 26 27.5) (end 40.88 27.5) (width 0.5) (layer "B.Cu") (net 7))
 (segment (start 26 65.5) (end 22.5 62) (width 0.5) (layer "B.Cu") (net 7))
 (segment (start 76.5 38.5) (end 65.5 27.5) (width 0.5) (layer "B.Cu") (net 2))
 (segment (start 70.5 93) (end 76.5 87) (width 0.5) (layer "B.Cu") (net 2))
 (segment (start 22 84.5) (end 22 93) (width 0.5) (layer "B.Cu") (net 2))
 (segment (start 22 93) (end 70.5 93) (width 0.5) (layer "B.Cu") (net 2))
 (segment (start 76.5 87) (end 76.5 38.5) (width 0.5) (layer "B.Cu") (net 2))
 (segment (start 65.5 27.5) (end 56.12 27.5) (width 0.5) (layer "B.Cu") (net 2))
 (segment (start 26 84.5) (end 22 84.5) (width 0.5) (layer "B.Cu") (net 2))
 (segment (start 40.88 40.38) (end 40.88 35.12) (width 0.5) (layer "B.Cu") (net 9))
 (segment (start 45.11 44.61) (end 40.88 40.38) (width 0.5) (layer "B.Cu") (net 9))
 (segment (start 45.11 46.46) (end 45.11 44.61) (width 0.5) (layer "B.Cu") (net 9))
 (segment (start 52 32.5) (end 52.08 32.58) (width 0.5) (layer "B.Cu") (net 11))
 (segment (start 52.08 32.58) (end 56.12 32.58) (width 0.5) (layer "B.Cu") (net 11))
 (segment (start 45.11 65.46) (end 45.11 61.39) (width 0.5) (layer "B.Cu") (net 11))
 (segment (start 51.5 38) (end 51.5 33) (width 0.5) (layer "B.Cu") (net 11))
 (segment (start 57 40) (end 57 42) (width 0.5) (layer "B.Cu") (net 11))
 (segment (start 57 56.5) (end 57 40) (width 0.5) (layer "B.Cu") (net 11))
 (segment (start 51.5 33) (end 52 32.5) (width 0.5) (layer "B.Cu") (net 11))
 (segment (start 48 58.5) (end 55 58.5) (width 0.5) (layer "B.Cu") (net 11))
 (segment (start 45.11 61.39) (end 48 58.5) (width 0.5) (layer "B.Cu") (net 11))
 (segment (start 55 58.5) (end 57 56.5) (width 0.5) (layer "B.Cu") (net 11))
 (segment (start 53.5 40) (end 51.5 38) (width 0.5) (layer "B.Cu") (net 11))
 (segment (start 57 40) (end 53.5 40) (width 0.5) (layer "B.Cu") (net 11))
 (segment (start 59.5 36.5) (end 59.5 71.5) (width 0.5) (layer "B.Cu") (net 10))
 (segment (start 59.5 71.5) (end 53 78) (width 0.5) (layer "B.Cu") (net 10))
 (segment (start 45 81.5) (end 45 84.5) (width 0.5) (layer "B.Cu") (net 10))
 (segment (start 53 78) (end 48.5 78) (width 0.5) (layer "B.Cu") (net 10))
 (segment (start 56.12 35.12) (end 58.12 35.12) (width 0.5) (layer "B.Cu") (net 10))
 (segment (start 48.5 78) (end 45 81.5) (width 0.5) (layer "B.Cu") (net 10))
 (segment (start 58.12 35.12) (end 59.5 36.5) (width 0.5) (layer "B.Cu") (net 10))
 (segment (start 64.11 31.11) (end 63 30) (width 0.5) (layer "B.Cu") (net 12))
 (segment (start 57.46 30.04) (end 56.12 30.04) (width 0.5) (layer "B.Cu") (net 12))
 (segment (start 63 30) (end 57.5 30) (width 0.5) (layer "B.Cu") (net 12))
 (segment (start 57.5 30) (end 57.46 30.04) (width 0.5) (layer "B.Cu") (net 12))
 (segment (start 64.11 46.46) (end 64.11 31.11) (width 0.5) (layer "B.Cu") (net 12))
 (segment (start 44.483 31.517) (end 43.42 32.58) (width 0.2) (layer "B.Cu") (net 3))
 (segment (start 64.11 65.46) (end 60.051 61.401) (width 0.2) (layer "B.Cu") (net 3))
 (segment (start 56.56031 31.517) (end 44.483 31.517) (width 0.2) (layer "B.Cu") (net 3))
 (segment (start 43.42 32.58) (end 40.88 32.58) (width 0.2) (layer "B.Cu") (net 3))
 (segment (start 60.051 35.00769) (end 56.56031 31.517) (width 0.2) (layer "B.Cu") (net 3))
 (segment (start 60.051 61.401) (end 60.051 35.00769) (width 0.2) (layer "B.Cu") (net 3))
 (segment (start 36.5 84.5) (end 32 84.5) (width 0.5) (layer "B.Cu") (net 6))
 (segment (start 21 27.5) (end 23.54 24.96) (width 0.5) (layer "B.Cu") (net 6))
 (segment (start 21 73.5) (end 21 27.5) (width 0.5) (layer "B.Cu") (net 6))
 (segment (start 58 87) (end 58 90) (width 0.5) (layer "B.Cu") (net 6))
 (segment (start 64 84.5) (end 60.5 84.5) (width 0.5) (layer "B.Cu") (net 6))
 (segment (start 58 90) (end 42 90) (width 0.5) (layer "B.Cu") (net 6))
 (segment (start 23.54 24.96) (end 40.88 24.96) (width 0.5) (layer "B.Cu") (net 6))
 (segment (start 32 84.5) (end 21 73.5) (width 0.5) (layer "B.Cu") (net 6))
 (segment (start 60.5 84.5) (end 58 87) (width 0.5) (layer "B.Cu") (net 6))
 (segment (start 42 90) (end 36.5 84.5) (width 0.5) (layer "B.Cu") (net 6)))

